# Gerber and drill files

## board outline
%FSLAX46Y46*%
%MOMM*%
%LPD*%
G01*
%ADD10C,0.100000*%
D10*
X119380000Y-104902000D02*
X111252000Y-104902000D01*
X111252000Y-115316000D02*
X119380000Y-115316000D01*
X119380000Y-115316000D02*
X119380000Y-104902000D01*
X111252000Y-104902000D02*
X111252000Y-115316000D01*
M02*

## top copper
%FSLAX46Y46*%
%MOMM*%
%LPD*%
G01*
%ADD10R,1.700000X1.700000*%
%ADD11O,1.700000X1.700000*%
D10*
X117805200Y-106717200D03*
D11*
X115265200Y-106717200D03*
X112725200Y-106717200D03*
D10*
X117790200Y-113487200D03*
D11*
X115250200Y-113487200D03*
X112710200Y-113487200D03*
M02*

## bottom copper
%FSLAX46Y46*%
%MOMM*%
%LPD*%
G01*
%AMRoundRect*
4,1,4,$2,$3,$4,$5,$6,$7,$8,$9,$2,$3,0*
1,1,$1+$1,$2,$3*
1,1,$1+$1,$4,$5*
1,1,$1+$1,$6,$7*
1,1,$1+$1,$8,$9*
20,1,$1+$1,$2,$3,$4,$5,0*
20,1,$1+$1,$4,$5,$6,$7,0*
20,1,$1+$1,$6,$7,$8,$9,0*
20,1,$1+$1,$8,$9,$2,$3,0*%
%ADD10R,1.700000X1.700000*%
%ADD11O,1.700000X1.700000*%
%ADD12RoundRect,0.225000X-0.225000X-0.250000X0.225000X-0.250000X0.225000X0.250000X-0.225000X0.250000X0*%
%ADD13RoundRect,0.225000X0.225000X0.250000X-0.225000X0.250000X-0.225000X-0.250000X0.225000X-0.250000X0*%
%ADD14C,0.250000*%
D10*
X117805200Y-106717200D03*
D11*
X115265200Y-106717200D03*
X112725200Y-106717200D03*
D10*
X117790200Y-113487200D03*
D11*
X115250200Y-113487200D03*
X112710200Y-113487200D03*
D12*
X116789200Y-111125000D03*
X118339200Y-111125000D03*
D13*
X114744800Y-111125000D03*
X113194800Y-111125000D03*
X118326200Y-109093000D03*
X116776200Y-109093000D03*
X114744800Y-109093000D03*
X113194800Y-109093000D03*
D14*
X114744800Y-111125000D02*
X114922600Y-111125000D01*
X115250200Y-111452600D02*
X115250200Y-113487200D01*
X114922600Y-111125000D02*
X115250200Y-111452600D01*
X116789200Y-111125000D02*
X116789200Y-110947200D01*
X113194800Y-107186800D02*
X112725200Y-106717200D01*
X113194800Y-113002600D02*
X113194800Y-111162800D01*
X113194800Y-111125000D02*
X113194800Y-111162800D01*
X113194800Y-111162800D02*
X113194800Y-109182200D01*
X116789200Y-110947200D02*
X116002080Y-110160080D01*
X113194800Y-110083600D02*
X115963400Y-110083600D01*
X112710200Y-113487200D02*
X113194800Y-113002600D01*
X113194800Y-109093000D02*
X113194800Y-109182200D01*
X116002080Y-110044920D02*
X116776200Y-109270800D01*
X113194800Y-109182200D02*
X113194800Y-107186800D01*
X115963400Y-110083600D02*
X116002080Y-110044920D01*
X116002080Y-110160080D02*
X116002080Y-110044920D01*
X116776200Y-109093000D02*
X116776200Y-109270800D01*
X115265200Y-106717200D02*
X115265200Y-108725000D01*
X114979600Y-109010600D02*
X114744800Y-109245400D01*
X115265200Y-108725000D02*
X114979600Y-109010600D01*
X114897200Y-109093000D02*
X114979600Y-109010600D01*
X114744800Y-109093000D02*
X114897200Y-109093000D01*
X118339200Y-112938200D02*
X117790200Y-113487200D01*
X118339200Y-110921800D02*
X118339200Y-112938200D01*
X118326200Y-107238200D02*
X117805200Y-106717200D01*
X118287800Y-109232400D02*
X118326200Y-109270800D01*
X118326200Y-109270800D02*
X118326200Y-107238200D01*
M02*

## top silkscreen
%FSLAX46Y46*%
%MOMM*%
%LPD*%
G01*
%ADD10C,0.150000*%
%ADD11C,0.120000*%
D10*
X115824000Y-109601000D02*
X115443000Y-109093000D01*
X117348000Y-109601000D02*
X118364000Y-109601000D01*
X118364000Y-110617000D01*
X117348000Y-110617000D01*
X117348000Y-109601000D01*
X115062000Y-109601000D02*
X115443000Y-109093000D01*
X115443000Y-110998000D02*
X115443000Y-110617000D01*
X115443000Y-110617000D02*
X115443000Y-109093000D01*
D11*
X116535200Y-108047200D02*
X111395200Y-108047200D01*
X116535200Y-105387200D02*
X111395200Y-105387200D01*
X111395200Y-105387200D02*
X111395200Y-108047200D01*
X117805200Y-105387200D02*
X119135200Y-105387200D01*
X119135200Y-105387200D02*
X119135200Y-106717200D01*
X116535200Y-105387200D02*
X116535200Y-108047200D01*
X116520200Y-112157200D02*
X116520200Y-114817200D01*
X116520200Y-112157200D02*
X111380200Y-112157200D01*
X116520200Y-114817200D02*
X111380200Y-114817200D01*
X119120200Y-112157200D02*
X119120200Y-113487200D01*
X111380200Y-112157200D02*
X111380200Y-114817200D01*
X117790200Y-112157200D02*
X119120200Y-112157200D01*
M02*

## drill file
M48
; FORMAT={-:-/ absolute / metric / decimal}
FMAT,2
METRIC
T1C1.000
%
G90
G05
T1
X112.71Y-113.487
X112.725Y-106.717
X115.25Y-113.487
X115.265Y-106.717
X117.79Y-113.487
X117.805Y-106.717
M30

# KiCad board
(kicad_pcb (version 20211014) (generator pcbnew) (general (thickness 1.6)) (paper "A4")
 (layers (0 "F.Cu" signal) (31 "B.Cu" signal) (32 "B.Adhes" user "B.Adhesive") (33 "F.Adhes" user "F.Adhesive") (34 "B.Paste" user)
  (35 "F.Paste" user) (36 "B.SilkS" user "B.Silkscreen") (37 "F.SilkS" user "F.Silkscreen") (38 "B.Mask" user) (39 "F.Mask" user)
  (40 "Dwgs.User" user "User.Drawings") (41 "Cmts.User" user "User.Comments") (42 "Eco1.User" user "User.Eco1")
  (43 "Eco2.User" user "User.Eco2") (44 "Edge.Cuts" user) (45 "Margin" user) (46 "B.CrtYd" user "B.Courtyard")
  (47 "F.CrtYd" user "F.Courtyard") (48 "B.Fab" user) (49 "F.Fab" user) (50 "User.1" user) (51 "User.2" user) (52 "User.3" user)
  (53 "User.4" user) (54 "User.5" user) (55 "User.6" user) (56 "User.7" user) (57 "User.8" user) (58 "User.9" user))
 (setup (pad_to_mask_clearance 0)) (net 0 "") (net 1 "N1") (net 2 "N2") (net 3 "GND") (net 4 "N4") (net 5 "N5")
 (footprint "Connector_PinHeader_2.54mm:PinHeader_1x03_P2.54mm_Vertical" (layer "F.Cu") (at 117.8052 106.7172 -90)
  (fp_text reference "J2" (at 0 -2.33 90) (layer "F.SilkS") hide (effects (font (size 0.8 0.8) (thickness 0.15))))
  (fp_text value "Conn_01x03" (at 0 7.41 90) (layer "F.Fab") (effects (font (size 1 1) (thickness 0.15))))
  (fp_line (start 1.33 1.27) (end 1.33 6.41) (layer "F.SilkS") (width 0.12))
  (fp_line (start -1.33 1.27) (end -1.33 6.41) (layer "F.SilkS") (width 0.12))
  (fp_line (start -1.33 6.41) (end 1.33 6.41) (layer "F.SilkS") (width 0.12))
  (fp_line (start -1.33 0) (end -1.33 -1.33) (layer "F.SilkS") (width 0.12))
  (fp_line (start -1.33 -1.33) (end 0 -1.33) (layer "F.SilkS") (width 0.12))
  (fp_line (start -1.33 1.27) (end 1.33 1.27) (layer "F.SilkS") (width 0.12))
  (pad "1" thru_hole rect (at 0 0 270) (size 1.7 1.7) (drill 1) (layers *.Cu *.Mask) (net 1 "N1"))
  (pad "2" thru_hole oval (at 0 2.54 270) (size 1.7 1.7) (drill 1) (layers *.Cu *.Mask) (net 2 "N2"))
  (pad "3" thru_hole oval (at 0 5.08 270) (size 1.7 1.7) (drill 1) (layers *.Cu *.Mask) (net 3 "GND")))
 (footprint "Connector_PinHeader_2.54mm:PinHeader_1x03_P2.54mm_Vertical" (layer "F.Cu") (at 117.7902 113.4872 -90)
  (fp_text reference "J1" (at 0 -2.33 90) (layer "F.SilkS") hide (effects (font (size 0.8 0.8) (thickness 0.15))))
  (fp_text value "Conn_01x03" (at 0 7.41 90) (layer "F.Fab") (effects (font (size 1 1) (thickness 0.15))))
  (fp_line (start -1.33 1.27) (end 1.33 1.27) (layer "F.SilkS") (width 0.12))
  (fp_line (start -1.33 1.27) (end -1.33 6.41) (layer "F.SilkS") (width 0.12))
  (fp_line (start 1.33 1.27) (end 1.33 6.41) (layer "F.SilkS") (width 0.12))
  (fp_line (start -1.33 -1.33) (end 0 -1.33) (layer "F.SilkS") (width 0.12))
  (fp_line (start -1.33 6.41) (end 1.33 6.41) (layer "F.SilkS") (width 0.12))
  (fp_line (start -1.33 0) (end -1.33 -1.33) (layer "F.SilkS") (width 0.12))
  (pad "1" thru_hole rect (at 0 0 270) (size 1.7 1.7) (drill 1) (layers *.Cu *.Mask) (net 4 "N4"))
  (pad "2" thru_hole oval (at 0 2.54 270) (size 1.7 1.7) (drill 1) (layers *.Cu *.Mask) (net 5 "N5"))
  (pad "3" thru_hole oval (at 0 5.08 270) (size 1.7 1.7) (drill 1) (layers *.Cu *.Mask) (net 3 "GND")))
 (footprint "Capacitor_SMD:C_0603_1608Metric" (layer "B.Cu") (at 117.5642 111.125)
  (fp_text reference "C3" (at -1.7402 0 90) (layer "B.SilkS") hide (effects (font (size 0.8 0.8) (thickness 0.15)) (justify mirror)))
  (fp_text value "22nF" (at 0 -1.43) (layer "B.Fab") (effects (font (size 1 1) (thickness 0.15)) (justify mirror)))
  (pad "1" smd roundrect (at -0.775 0) (size 0.9 0.95) (layers "B.Cu" "B.Paste" "B.Mask") (roundrect_rratio 0.25) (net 3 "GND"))
  (pad "2" smd roundrect (at 0.775 0) (size 0.9 0.95) (layers "B.Cu" "B.Paste" "B.Mask") (roundrect_rratio 0.25) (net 4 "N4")))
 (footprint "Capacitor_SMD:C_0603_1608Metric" (layer "B.Cu") (at 113.9698 111.125 180)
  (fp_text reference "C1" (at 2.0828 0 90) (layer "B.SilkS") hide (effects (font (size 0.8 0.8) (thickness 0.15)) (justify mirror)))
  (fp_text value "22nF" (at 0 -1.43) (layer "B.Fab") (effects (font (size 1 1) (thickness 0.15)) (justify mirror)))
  (pad "1" smd roundrect (at -0.775 0 180) (size 0.9 0.95) (layers "B.Cu" "B.Paste" "B.Mask") (roundrect_rratio 0.25) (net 5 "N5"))
  (pad "2" smd roundrect (at 0.775 0 180) (size 0.9 0.95) (layers "B.Cu" "B.Paste" "B.Mask") (roundrect_rratio 0.25) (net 3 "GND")))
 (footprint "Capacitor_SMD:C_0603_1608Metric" (layer "B.Cu") (at 117.5512 109.093 180)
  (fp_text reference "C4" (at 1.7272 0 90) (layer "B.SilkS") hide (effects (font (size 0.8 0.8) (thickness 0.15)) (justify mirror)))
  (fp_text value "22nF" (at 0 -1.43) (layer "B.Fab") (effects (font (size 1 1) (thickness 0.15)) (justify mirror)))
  (pad "1" smd roundrect (at -0.775 0 180) (size 0.9 0.95) (layers "B.Cu" "B.Paste" "B.Mask") (roundrect_rratio 0.25) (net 1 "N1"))
  (pad "2" smd roundrect (at 0.775 0 180) (size 0.9 0.95) (layers "B.Cu" "B.Paste" "B.Mask") (roundrect_rratio 0.25) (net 3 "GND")))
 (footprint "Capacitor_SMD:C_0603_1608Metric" (layer "B.Cu") (at 113.9698 109.093 180)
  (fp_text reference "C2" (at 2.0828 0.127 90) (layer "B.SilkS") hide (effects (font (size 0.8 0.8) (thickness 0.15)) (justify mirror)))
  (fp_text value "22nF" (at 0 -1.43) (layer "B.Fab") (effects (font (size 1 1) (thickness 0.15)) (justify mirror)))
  (pad "1" smd roundrect (at -0.775 0 180) (size 0.9 0.95) (layers "B.Cu" "B.Paste" "B.Mask") (roundrect_rratio 0.25) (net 2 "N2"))
  (pad "2" smd roundrect (at 0.775 0 180) (size 0.9 0.95) (layers "B.Cu" "B.Paste" "B.Mask") (roundrect_rratio 0.25) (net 3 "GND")))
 (gr_line (start 115.824 109.601) (end 115.443 109.093) (layer "F.SilkS") (width 0.15))
 (gr_rect (start 117.348 109.601) (end 118.364 110.617) (layer "F.SilkS") (width 0.15) (fill none))
 (gr_line (start 115.062 109.601) (end 115.443 109.093) (layer "F.SilkS") (width 0.15))
 (gr_line (start 115.443 110.998) (end 115.443 110.617) (layer "F.SilkS") (width 0.15))
 (gr_line (start 115.443 110.617) (end 115.443 109.093) (layer "F.SilkS") (width 0.15))
 (gr_line (start 119.38 104.902) (end 111.252 104.902) (layer "Edge.Cuts") (width 0.1))
 (gr_line (start 111.252 115.316) (end 119.38 115.316) (layer "Edge.Cuts") (width 0.1))
 (gr_line (start 119.38 115.316) (end 119.38 104.902) (layer "Edge.Cuts") (width 0.1))
 (gr_line (start 111.252 104.902) (end 111.252 115.316) (layer "Edge.Cuts") (width 0.1))
 (segment (start 114.7448 111.125) (end 114.9226 111.125) (width 0.25) (layer "B.Cu") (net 5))
 (segment (start 115.2502 111.4526) (end 115.2502 113.4872) (width 0.25) (layer "B.Cu") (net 5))
 (segment (start 114.9226 111.125) (end 115.2502 111.4526) (width 0.25) (layer "B.Cu") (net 5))
 (segment (start 116.7892 111.125) (end 116.7892 110.9472) (width 0.25) (layer "B.Cu") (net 3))
 (segment (start 113.1948 107.1868) (end 112.7252 106.7172) (width 0.25) (layer "B.Cu") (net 3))
 (segment (start 113.1948 113.0026) (end 113.1948 111.1628) (width 0.25) (layer "B.Cu") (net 3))
 (segment (start 113.1948 111.125) (end 113.1948 111.1628) (width 0.25) (layer "B.Cu") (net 3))
 (segment (start 113.1948 111.1628) (end 113.1948 109.1822) (width 0.25) (layer "B.Cu") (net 3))
 (segment (start 116.7892 110.9472) (end 116.00208 110.16008) (width 0.25) (layer "B.Cu") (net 3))
 (segment (start 113.1948 110.0836) (end 115.9634 110.0836) (width 0.25) (layer "B.Cu") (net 3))
 (segment (start 112.7102 113.4872) (end 113.1948 113.0026) (width 0.25) (layer "B.Cu") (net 3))
 (segment (start 113.1948 109.093) (end 113.1948 109.1822) (width 0.25) (layer "B.Cu") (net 3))
 (segment (start 116.00208 110.04492) (end 116.7762 109.2708) (width 0.25) (layer "B.Cu") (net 3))
 (segment (start 113.1948 109.1822) (end 113.1948 107.1868) (width 0.25) (layer "B.Cu") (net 3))
 (segment (start 115.9634 110.0836) (end 116.00208 110.04492) (width 0.25) (layer "B.Cu") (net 3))
 (segment (start 116.00208 110.16008) (end 116.00208 110.04492) (width 0.25) (layer "B.Cu") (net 3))
 (segment (start 116.7762 109.093) (end 116.7762 109.2708) (width 0.25) (layer "B.Cu") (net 3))
 (segment (start 115.2652 106.7172) (end 115.2652 108.725) (width 0.25) (layer "B.Cu") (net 2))
 (segment (start 114.9796 109.0106) (end 114.7448 109.2454) (width 0.25) (layer "B.Cu") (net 2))
 (segment (start 115.2652 108.725) (end 114.9796 109.0106) (width 0.25) (layer "B.Cu") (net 2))
 (segment (start 114.8972 109.093) (end 114.9796 109.0106) (width 0.25) (layer "B.Cu") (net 2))
 (segment (start 114.7448 109.093) (end 114.8972 109.093) (width 0.25) (layer "B.Cu") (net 2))
 (segment (start 118.3392 112.9382) (end 117.7902 113.4872) (width 0.25) (layer "B.Cu") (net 4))
 (segment (start 118.3392 110.9218) (end 118.3392 112.9382) (width 0.25) (layer "B.Cu") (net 4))
 (segment (start 118.3262 107.2382) (end 117.8052 106.7172) (width 0.25) (layer "B.Cu") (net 1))
 (segment (start 118.2878 109.2324) (end 118.3262 109.2708) (width 0.25) (layer "B.Cu") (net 1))
 (segment (start 118.3262 109.2708) (end 118.3262 107.2382) (width 0.25) (layer "B.Cu") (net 1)))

